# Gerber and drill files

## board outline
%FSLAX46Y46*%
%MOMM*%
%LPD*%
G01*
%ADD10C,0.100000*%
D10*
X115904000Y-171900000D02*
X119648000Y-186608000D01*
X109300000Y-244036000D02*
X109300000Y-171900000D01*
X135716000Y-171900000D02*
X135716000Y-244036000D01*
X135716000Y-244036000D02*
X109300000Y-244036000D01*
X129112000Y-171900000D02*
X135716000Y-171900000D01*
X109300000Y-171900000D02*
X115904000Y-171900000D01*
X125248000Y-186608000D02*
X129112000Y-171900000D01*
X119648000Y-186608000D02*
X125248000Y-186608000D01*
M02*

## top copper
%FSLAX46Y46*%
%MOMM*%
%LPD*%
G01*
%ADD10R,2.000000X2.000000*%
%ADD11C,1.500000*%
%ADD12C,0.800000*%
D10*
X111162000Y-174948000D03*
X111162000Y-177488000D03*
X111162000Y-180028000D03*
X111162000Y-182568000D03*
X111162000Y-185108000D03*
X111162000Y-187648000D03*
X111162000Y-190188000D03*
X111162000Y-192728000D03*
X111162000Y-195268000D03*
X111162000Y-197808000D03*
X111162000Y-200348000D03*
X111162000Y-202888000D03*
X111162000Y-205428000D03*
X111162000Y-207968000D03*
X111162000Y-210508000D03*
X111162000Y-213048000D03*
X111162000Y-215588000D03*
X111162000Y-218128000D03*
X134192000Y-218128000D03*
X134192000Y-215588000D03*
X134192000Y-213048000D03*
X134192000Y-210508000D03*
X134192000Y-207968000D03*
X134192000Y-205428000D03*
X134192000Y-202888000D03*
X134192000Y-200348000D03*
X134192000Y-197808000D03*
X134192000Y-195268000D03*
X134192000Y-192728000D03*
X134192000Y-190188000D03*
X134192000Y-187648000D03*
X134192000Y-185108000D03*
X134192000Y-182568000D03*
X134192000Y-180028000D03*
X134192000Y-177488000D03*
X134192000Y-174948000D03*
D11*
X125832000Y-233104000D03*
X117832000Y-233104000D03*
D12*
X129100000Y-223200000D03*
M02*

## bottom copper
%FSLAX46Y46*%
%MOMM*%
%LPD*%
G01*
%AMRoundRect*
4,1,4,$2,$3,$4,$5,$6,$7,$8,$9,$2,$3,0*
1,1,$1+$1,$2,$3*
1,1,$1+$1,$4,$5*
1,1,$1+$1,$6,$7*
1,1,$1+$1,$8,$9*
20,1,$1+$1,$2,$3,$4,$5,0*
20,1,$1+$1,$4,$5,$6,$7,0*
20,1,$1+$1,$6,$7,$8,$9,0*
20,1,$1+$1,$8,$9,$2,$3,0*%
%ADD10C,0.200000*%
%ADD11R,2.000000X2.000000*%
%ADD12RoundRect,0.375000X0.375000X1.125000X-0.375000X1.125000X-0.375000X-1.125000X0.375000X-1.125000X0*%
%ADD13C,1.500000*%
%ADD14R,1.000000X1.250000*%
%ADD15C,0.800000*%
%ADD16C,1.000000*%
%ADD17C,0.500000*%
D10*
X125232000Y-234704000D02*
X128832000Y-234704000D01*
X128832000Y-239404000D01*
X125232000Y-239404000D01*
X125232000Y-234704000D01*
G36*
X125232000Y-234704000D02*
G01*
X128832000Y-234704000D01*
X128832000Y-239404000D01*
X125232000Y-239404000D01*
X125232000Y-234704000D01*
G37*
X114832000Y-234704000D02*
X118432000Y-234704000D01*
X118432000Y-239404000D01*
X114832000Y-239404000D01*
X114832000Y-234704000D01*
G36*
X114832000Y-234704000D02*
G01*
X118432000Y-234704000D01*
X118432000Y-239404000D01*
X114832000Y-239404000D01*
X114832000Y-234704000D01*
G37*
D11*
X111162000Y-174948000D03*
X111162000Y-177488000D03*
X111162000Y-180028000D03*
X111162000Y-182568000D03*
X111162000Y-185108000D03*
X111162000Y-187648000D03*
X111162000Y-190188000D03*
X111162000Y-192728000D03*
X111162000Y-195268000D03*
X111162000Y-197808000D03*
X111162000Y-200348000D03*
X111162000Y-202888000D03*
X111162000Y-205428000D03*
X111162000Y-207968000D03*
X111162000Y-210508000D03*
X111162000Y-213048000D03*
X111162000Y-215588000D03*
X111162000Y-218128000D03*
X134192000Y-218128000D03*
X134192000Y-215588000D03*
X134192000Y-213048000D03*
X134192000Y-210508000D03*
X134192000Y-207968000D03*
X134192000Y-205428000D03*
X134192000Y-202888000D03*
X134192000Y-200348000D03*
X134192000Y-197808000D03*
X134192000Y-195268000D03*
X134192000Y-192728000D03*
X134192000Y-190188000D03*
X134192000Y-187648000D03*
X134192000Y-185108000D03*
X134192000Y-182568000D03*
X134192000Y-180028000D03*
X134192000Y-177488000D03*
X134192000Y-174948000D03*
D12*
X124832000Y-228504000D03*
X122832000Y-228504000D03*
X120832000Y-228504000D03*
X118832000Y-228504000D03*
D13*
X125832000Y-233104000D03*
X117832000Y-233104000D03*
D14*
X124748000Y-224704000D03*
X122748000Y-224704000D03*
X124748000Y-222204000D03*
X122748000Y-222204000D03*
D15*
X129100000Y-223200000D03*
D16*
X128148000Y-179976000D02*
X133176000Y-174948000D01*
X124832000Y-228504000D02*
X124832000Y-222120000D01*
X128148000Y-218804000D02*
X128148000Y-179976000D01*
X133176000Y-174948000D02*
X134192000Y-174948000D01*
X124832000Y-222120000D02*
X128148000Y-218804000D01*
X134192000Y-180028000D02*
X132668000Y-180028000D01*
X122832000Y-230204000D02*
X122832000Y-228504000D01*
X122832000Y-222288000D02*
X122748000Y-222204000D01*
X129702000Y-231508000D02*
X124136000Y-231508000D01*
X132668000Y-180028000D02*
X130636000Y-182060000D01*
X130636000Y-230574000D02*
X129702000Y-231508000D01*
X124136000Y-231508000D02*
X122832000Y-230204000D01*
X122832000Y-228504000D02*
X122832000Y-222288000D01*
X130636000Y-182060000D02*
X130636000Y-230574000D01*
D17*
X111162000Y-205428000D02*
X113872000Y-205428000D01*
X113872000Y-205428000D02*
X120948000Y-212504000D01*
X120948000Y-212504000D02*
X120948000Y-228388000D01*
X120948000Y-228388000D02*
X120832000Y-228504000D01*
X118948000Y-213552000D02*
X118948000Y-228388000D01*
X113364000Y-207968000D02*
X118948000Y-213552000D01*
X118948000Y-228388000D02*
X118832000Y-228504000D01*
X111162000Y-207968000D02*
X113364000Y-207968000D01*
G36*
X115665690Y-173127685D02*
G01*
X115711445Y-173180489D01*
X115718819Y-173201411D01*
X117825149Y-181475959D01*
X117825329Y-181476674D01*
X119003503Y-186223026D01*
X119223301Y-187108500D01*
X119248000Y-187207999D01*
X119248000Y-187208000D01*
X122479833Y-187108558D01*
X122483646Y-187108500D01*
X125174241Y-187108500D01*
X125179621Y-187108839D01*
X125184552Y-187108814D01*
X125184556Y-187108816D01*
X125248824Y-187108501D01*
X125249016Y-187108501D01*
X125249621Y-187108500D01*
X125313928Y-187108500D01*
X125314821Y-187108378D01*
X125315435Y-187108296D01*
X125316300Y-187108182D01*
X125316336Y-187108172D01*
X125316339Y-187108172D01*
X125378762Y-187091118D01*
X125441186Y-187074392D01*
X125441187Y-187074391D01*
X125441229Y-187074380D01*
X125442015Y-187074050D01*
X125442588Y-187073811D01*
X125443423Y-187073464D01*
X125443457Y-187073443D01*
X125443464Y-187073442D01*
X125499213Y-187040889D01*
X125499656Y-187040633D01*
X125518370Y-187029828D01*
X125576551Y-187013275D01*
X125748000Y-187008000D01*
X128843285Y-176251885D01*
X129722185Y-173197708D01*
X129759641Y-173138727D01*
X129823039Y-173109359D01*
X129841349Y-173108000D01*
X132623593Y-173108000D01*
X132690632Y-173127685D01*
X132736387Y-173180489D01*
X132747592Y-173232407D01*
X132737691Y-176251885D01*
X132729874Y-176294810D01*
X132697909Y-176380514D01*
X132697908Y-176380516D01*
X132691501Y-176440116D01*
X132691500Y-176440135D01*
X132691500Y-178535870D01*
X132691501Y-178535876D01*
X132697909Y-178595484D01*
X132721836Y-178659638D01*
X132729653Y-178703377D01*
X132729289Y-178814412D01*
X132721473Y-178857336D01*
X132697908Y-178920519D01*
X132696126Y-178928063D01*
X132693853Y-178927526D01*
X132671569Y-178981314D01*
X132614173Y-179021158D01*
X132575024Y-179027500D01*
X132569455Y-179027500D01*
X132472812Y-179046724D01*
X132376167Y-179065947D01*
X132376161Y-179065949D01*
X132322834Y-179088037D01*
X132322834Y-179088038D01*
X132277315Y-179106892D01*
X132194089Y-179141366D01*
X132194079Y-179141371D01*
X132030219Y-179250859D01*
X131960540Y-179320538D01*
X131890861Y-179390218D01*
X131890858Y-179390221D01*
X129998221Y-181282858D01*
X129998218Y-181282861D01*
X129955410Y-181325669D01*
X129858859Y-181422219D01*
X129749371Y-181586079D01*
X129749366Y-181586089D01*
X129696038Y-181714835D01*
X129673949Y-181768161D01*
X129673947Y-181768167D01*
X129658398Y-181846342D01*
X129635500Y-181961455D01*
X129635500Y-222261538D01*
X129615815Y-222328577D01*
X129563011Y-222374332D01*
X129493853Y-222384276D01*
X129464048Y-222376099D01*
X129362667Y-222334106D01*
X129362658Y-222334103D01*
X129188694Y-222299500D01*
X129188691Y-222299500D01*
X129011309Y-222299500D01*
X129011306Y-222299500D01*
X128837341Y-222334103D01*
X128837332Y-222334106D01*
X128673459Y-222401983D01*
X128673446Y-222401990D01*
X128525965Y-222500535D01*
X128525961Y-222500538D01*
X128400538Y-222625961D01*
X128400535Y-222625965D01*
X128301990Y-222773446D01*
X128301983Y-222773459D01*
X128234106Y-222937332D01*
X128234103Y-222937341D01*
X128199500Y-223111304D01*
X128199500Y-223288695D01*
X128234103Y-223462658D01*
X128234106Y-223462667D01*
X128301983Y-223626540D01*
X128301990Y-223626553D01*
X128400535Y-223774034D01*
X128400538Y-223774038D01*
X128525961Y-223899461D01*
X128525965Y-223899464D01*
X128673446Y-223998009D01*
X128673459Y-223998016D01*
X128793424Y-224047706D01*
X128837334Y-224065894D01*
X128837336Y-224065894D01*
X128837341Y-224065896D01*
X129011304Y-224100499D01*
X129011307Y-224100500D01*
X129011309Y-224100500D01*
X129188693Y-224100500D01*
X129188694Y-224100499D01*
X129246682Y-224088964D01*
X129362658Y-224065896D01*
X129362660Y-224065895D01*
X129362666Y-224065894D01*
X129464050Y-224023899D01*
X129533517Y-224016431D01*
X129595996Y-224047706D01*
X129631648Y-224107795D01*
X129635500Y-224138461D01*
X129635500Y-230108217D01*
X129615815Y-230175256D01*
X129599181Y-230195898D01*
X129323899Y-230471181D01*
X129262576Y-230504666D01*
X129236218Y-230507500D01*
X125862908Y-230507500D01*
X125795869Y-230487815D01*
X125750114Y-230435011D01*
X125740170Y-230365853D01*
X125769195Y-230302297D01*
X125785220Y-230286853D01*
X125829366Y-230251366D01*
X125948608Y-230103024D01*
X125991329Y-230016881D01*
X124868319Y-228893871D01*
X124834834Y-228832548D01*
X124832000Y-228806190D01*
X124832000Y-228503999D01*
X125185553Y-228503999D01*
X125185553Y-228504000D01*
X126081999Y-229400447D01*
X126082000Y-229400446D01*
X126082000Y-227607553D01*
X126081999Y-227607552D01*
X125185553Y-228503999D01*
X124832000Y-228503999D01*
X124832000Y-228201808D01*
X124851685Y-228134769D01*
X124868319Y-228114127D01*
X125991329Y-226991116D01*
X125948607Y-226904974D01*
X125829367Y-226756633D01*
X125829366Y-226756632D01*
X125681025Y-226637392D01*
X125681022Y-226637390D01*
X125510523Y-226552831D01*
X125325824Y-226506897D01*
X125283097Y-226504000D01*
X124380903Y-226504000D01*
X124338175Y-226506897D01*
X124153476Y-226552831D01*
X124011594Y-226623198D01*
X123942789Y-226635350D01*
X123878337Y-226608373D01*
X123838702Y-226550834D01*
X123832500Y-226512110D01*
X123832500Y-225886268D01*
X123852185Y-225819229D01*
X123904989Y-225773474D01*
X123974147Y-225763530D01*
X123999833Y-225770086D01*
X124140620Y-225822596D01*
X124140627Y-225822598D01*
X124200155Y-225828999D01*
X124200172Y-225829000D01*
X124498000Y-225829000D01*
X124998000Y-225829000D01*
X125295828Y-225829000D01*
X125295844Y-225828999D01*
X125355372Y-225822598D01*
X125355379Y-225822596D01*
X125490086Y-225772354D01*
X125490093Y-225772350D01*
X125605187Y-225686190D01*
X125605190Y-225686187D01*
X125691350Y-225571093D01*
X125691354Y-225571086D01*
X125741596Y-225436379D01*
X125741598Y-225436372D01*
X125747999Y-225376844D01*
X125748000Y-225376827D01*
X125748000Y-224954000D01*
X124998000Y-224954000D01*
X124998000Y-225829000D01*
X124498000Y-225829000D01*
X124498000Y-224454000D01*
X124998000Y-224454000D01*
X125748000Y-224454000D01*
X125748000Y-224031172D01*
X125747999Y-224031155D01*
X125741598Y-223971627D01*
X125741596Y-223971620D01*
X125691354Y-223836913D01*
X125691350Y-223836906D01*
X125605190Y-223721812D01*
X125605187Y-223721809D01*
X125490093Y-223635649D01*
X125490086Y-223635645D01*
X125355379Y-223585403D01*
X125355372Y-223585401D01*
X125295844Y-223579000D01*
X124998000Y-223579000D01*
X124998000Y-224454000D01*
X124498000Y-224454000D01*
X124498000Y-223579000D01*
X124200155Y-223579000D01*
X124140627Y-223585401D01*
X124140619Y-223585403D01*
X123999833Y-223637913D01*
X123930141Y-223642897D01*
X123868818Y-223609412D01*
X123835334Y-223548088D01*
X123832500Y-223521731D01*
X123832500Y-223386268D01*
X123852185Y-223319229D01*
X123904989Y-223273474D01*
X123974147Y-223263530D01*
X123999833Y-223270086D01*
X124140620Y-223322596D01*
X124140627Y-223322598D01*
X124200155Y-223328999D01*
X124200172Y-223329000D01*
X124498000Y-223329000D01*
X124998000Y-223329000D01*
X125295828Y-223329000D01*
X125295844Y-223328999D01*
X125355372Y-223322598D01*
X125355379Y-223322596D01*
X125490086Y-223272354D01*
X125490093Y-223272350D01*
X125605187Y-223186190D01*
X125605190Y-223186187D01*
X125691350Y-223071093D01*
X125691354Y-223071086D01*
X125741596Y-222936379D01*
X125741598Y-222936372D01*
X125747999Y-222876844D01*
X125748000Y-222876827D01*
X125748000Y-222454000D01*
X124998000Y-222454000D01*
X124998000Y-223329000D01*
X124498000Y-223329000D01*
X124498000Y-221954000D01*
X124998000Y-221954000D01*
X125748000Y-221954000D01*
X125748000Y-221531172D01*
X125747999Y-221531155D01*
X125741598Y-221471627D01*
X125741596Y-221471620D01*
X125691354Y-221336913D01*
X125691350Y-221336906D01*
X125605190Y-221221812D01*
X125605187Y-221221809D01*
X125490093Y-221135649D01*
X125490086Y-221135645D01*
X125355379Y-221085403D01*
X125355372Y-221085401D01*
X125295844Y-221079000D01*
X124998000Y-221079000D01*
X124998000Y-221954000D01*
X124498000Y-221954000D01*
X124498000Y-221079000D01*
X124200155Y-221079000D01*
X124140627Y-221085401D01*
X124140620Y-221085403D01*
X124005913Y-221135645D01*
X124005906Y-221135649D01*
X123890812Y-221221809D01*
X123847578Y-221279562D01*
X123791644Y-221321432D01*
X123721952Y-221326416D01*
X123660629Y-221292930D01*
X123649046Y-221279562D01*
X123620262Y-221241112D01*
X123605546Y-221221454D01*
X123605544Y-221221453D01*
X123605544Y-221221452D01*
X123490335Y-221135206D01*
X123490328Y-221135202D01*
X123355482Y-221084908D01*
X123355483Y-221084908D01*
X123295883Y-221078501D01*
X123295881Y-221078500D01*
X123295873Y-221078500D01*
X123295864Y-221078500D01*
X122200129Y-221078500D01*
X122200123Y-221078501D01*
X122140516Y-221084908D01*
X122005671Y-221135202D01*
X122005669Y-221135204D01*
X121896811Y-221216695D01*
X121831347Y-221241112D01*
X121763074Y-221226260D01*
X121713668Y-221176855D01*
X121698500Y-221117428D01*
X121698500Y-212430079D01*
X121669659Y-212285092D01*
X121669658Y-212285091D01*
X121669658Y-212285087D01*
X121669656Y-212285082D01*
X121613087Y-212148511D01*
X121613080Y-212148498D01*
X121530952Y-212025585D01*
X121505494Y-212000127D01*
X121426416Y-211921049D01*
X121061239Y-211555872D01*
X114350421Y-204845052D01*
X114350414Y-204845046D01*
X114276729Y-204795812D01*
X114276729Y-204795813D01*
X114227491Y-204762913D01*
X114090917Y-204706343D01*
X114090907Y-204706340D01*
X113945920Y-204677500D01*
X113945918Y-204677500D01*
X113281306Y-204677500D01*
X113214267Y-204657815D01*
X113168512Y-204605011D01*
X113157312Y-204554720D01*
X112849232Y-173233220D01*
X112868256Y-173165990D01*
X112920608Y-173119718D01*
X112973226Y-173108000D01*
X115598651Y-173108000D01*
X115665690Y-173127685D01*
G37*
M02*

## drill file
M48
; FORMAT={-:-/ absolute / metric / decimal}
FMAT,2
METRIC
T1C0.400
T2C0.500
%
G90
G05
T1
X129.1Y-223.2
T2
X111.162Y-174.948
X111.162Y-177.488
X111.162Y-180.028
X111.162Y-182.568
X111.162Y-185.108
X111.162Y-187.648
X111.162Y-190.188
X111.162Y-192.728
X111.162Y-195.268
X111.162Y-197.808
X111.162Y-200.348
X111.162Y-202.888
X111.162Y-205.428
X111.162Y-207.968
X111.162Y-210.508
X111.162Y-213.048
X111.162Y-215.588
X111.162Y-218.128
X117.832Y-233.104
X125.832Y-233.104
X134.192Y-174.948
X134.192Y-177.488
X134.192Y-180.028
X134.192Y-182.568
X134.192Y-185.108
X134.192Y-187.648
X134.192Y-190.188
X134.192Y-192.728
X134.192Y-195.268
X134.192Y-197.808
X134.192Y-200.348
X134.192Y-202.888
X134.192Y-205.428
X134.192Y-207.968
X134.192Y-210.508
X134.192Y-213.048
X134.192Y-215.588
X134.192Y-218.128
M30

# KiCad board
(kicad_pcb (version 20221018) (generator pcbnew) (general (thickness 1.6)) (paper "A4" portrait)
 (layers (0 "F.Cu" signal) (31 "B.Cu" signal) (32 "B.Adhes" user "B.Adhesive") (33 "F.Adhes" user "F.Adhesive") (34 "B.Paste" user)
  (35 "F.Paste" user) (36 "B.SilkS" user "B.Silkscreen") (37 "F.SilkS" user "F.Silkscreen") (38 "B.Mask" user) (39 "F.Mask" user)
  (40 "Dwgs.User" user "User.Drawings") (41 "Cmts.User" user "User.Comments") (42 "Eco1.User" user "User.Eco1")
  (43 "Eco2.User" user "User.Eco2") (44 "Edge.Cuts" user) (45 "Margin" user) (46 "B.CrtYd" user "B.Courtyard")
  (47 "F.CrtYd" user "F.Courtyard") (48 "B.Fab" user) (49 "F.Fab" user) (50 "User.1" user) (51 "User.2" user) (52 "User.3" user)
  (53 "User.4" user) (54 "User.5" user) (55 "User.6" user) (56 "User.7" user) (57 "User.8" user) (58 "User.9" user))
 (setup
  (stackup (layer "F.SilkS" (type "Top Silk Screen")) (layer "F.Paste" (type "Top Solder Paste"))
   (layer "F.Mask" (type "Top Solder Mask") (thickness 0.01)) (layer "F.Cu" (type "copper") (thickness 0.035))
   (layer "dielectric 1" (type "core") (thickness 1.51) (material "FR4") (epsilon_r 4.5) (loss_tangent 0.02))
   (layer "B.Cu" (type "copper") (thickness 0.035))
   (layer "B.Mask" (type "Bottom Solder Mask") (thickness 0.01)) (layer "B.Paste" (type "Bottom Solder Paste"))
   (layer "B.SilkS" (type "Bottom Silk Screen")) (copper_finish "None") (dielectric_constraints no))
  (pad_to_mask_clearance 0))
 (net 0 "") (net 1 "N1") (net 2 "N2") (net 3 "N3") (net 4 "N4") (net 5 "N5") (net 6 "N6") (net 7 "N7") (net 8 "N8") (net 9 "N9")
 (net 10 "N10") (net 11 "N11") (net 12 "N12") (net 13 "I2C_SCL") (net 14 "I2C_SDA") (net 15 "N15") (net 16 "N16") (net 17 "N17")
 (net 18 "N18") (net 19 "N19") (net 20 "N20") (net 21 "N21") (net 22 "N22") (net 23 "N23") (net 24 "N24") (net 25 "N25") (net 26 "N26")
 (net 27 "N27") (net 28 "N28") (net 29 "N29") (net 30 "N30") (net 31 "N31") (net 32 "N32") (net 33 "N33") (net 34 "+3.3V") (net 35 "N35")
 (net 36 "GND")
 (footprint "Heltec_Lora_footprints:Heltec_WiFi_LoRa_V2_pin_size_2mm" (layer "F.Cu") (at 122.677 200.348)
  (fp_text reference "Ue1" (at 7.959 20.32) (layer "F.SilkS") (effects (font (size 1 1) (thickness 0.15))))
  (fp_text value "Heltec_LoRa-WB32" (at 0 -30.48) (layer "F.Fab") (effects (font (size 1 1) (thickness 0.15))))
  (pad "1" thru_hole rect (at -11.515 -25.4) (size 2 2) (drill 0.5) (layers "*.Cu" "*.Mask") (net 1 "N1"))
  (pad "2" thru_hole rect (at -11.515 -22.86) (size 2 2) (drill 0.5) (layers "*.Cu" "*.Mask") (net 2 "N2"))
  (pad "3" thru_hole rect (at -11.515 -20.32) (size 2 2) (drill 0.5) (layers "*.Cu" "*.Mask") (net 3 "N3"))
  (pad "4" thru_hole rect (at -11.515 -17.78) (size 2 2) (drill 0.5) (layers "*.Cu" "*.Mask") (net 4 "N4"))
  (pad "5" thru_hole rect (at -11.515 -15.24) (size 2 2) (drill 0.5) (layers "*.Cu" "*.Mask") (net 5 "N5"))
  (pad "6" thru_hole rect (at -11.515 -12.7) (size 2 2) (drill 0.5) (layers "*.Cu" "*.Mask") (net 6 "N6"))
  (pad "7" thru_hole rect (at -11.515 -10.16) (size 2 2) (drill 0.5) (layers "*.Cu" "*.Mask") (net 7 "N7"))
  (pad "8" thru_hole rect (at -11.515 -7.62) (size 2 2) (drill 0.5) (layers "*.Cu" "*.Mask") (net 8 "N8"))
  (pad "9" thru_hole rect (at -11.515 -5.08) (size 2 2) (drill 0.5) (layers "*.Cu" "*.Mask") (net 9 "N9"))
  (pad "10" thru_hole rect (at -11.515 -2.54) (size 2 2) (drill 0.5) (layers "*.Cu" "*.Mask") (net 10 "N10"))
  (pad "11" thru_hole rect (at -11.515 0) (size 2 2) (drill 0.5) (layers "*.Cu" "*.Mask") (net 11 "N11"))
  (pad "12" thru_hole rect (at -11.515 2.54) (size 2 2) (drill 0.5) (layers "*.Cu" "*.Mask") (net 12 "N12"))
  (pad "13" thru_hole rect (at -11.515 5.08) (size 2 2) (drill 0.5) (layers "*.Cu" "*.Mask") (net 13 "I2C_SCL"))
  (pad "14" thru_hole rect (at -11.515 7.62) (size 2 2) (drill 0.5) (layers "*.Cu" "*.Mask") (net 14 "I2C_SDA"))
  (pad "15" thru_hole rect (at -11.515 10.16) (size 2 2) (drill 0.5) (layers "*.Cu" "*.Mask") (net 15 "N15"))
  (pad "16" thru_hole rect (at -11.515 12.7) (size 2 2) (drill 0.5) (layers "*.Cu" "*.Mask") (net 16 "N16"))
  (pad "17" thru_hole rect (at -11.515 15.24) (size 2 2) (drill 0.5) (layers "*.Cu" "*.Mask") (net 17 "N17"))
  (pad "18" thru_hole rect (at -11.515 17.78) (size 2 2) (drill 0.5) (layers "*.Cu" "*.Mask") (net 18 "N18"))
  (pad "19" thru_hole rect (at 11.515 17.78) (size 2 2) (drill 0.5) (layers "*.Cu" "*.Mask") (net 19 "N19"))
  (pad "20" thru_hole rect (at 11.515 15.24) (size 2 2) (drill 0.5) (layers "*.Cu" "*.Mask") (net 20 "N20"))
  (pad "21" thru_hole rect (at 11.515 12.7) (size 2 2) (drill 0.5) (layers "*.Cu" "*.Mask") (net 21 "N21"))
  (pad "22" thru_hole rect (at 11.515 10.16) (size 2 2) (drill 0.5) (layers "*.Cu" "*.Mask") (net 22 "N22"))
  (pad "23" thru_hole rect (at 11.515 7.62) (size 2 2) (drill 0.5) (layers "*.Cu" "*.Mask") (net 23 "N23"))
  (pad "24" thru_hole rect (at 11.515 5.08) (size 2 2) (drill 0.5) (layers "*.Cu" "*.Mask" "Eco2.User") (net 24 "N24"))
  (pad "25" thru_hole rect (at 11.515 2.54) (size 2 2) (drill 0.5) (layers "*.Cu" "*.Mask") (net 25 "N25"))
  (pad "26" thru_hole rect (at 11.515 0) (size 2 2) (drill 0.5) (layers "*.Cu" "*.Mask") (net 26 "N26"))
  (pad "27" thru_hole rect (at 11.515 -2.54) (size 2 2) (drill 0.5) (layers "*.Cu" "*.Mask") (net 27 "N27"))
  (pad "28" thru_hole rect (at 11.515 -5.08) (size 2 2) (drill 0.5) (layers "*.Cu" "*.Mask") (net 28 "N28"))
  (pad "29" thru_hole rect (at 11.515 -7.62) (size 2 2) (drill 0.5) (layers "*.Cu" "*.Mask") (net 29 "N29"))
  (pad "30" thru_hole rect (at 11.515 -10.16) (size 2 2) (drill 0.5) (layers "*.Cu" "*.Mask") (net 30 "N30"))
  (pad "31" thru_hole rect (at 11.515 -12.7) (size 2 2) (drill 0.5) (layers "*.Cu" "*.Mask") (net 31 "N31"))
  (pad "32" thru_hole rect (at 11.515 -15.24) (size 2 2) (drill 0.5) (layers "*.Cu" "*.Mask" "B.Paste") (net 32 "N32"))
  (pad "33" thru_hole rect (at 11.515 -17.78) (size 2 2) (drill 0.5) (layers "*.Cu" "*.Mask") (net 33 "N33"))
  (pad "34" thru_hole rect (at 11.515 -20.32) (size 2 2) (drill 0.5) (layers "*.Cu" "*.Mask") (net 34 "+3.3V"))
  (pad "35" thru_hole rect (at 11.515 -22.86) (size 2 2) (drill 0.5) (layers "*.Cu" "*.Mask") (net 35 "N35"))
  (pad "36" thru_hole rect (at 11.515 -25.4) (size 2 2) (drill 0.5) (layers "*.Cu" "*.Mask") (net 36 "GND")))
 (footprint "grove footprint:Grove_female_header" (layer "B.Cu") (at 121.832 234.604 180)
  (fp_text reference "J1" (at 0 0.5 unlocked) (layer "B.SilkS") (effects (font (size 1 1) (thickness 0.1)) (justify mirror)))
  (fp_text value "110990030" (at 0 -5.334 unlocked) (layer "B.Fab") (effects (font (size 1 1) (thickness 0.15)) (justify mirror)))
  (fp_rect (start -7 -0.1) (end -3.4 -4.8) (stroke (width 0.2) (type solid)) (fill solid) (layer "B.Cu"))
  (fp_rect (start 3.4 -0.1) (end 7 -4.8) (stroke (width 0.2) (type solid)) (fill solid) (layer "B.Cu"))
  (pad "1" smd roundrect (at -3 6.1 180) (size 1.5 3) (layers "B.Cu" "B.Paste" "B.Mask") (roundrect_rratio 0.25) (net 36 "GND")
   (thermal_bridge_angle 45))
  (pad "2" smd roundrect (at -1 6.1 180) (size 1.5 3) (layers "B.Cu" "B.Paste" "B.Mask") (roundrect_rratio 0.25) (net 34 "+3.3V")
   (thermal_bridge_angle 45))
  (pad "3" smd roundrect (at 1 6.1 180) (size 1.5 3) (layers "B.Cu" "B.Paste" "B.Mask") (roundrect_rratio 0.25) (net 13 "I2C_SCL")
   (thermal_bridge_angle 45))
  (pad "4" smd roundrect (at 3 6.1 180) (size 1.5 3) (layers "B.Cu" "B.Paste" "B.Mask") (roundrect_rratio 0.25) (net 14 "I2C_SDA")
   (thermal_bridge_angle 45))
  (pad "5" thru_hole circle (at -4 1.5 180) (size 1.5 1.5) (drill 0.5) (layers "*.Cu" "*.Mask"))
  (pad "5" thru_hole circle (at 4 1.5 180) (size 1.5 1.5) (drill 0.5) (layers "*.Cu" "*.Mask")))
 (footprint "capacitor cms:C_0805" (layer "B.Cu") (at 123.748 224.704 180)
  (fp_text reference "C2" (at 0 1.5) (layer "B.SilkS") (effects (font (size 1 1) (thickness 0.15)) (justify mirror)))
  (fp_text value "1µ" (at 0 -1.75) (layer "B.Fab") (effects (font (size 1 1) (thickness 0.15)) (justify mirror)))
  (pad "1" smd rect (at -1 0 180) (size 1 1.25) (layers "B.Cu" "B.Paste" "B.Mask") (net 36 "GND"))
  (pad "2" smd rect (at 1 0 180) (size 1 1.25) (layers "B.Cu" "B.Paste" "B.Mask") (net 34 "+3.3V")))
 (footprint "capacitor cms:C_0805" (layer "B.Cu") (at 123.748 222.204 180)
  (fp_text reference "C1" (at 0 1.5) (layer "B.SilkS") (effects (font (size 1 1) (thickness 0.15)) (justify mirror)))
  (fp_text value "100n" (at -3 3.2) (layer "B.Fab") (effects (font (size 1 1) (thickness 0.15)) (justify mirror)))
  (pad "1" smd rect (at -1 0 180) (size 1 1.25) (layers "B.Cu" "B.Paste" "B.Mask") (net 36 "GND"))
  (pad "2" smd rect (at 1 0 180) (size 1 1.25) (layers "B.Cu" "B.Paste" "B.Mask") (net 34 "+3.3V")))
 (gr_line (start 115.904 171.9) (end 119.648 186.608) (stroke (width 0.1) (type default)) (layer "Edge.Cuts"))
 (gr_line (start 109.3 244.036) (end 109.3 171.9) (stroke (width 0.1) (type default)) (layer "Edge.Cuts"))
 (gr_line (start 135.716 171.9) (end 135.716 244.036) (stroke (width 0.1) (type default)) (layer "Edge.Cuts"))
 (gr_line (start 135.716 244.036) (end 109.3 244.036) (stroke (width 0.1) (type default)) (layer "Edge.Cuts"))
 (gr_line (start 129.112 171.9) (end 135.716 171.9) (stroke (width 0.1) (type default)) (layer "Edge.Cuts"))
 (gr_line (start 109.3 171.9) (end 115.904 171.9) (stroke (width 0.1) (type default)) (layer "Edge.Cuts"))
 (gr_line (start 125.248 186.608) (end 129.112 171.9) (stroke (width 0.1) (type default)) (layer "Edge.Cuts"))
 (gr_line (start 119.648 186.608) (end 125.248 186.608) (stroke (width 0.1) (type default)) (layer "Edge.Cuts"))
 (via (at 129.1 223.2) (size 0.8) (drill 0.4) (layers "F.Cu" "B.Cu") (free) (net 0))
 (segment (start 128.148 179.976) (end 133.176 174.948) (width 1) (layer "B.Cu") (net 36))
 (segment (start 124.832 228.504) (end 124.832 222.12) (width 1) (layer "B.Cu") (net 36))
 (segment (start 128.148 218.804) (end 128.148 179.976) (width 1) (layer "B.Cu") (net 36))
 (segment (start 133.176 174.948) (end 134.192 174.948) (width 1) (layer "B.Cu") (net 36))
 (segment (start 124.832 222.12) (end 128.148 218.804) (width 1) (layer "B.Cu") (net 36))
 (segment (start 134.192 180.028) (end 132.668 180.028) (width 1) (layer "B.Cu") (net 34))
 (segment (start 122.832 230.204) (end 122.832 228.504) (width 1) (layer "B.Cu") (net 34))
 (segment (start 122.832 222.288) (end 122.748 222.204) (width 1) (layer "B.Cu") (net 34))
 (segment (start 129.702 231.508) (end 124.136 231.508) (width 1) (layer "B.Cu") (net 34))
 (segment (start 132.668 180.028) (end 130.636 182.06) (width 1) (layer "B.Cu") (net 34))
 (segment (start 130.636 230.574) (end 129.702 231.508) (width 1) (layer "B.Cu") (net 34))
 (segment (start 124.136 231.508) (end 122.832 230.204) (width 1) (layer "B.Cu") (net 34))
 (segment (start 122.832 228.504) (end 122.832 222.288) (width 1) (layer "B.Cu") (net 34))
 (segment (start 130.636 182.06) (end 130.636 230.574) (width 1) (layer "B.Cu") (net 34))
 (segment (start 111.162 205.428) (end 113.872 205.428) (width 0.5) (layer "B.Cu") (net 13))
 (segment (start 113.872 205.428) (end 120.948 212.504) (width 0.5) (layer "B.Cu") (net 13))
 (segment (start 120.948 212.504) (end 120.948 228.388) (width 0.5) (layer "B.Cu") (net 13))
 (segment (start 120.948 228.388) (end 120.832 228.504) (width 0.5) (layer "B.Cu") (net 13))
 (segment (start 118.948 213.552) (end 118.948 228.388) (width 0.5) (layer "B.Cu") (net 14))
 (segment (start 113.364 207.968) (end 118.948 213.552) (width 0.5) (layer "B.Cu") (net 14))
 (segment (start 118.948 228.388) (end 118.832 228.504) (width 0.5) (layer "B.Cu") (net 14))
 (segment (start 111.162 207.968) (end 113.364 207.968) (width 0.5) (layer "B.Cu") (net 14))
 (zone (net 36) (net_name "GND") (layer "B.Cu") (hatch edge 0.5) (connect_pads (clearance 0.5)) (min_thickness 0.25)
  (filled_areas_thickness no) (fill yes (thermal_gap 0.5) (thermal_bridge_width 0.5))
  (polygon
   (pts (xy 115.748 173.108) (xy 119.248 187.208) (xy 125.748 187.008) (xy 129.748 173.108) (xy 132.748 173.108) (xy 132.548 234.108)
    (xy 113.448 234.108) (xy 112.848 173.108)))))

